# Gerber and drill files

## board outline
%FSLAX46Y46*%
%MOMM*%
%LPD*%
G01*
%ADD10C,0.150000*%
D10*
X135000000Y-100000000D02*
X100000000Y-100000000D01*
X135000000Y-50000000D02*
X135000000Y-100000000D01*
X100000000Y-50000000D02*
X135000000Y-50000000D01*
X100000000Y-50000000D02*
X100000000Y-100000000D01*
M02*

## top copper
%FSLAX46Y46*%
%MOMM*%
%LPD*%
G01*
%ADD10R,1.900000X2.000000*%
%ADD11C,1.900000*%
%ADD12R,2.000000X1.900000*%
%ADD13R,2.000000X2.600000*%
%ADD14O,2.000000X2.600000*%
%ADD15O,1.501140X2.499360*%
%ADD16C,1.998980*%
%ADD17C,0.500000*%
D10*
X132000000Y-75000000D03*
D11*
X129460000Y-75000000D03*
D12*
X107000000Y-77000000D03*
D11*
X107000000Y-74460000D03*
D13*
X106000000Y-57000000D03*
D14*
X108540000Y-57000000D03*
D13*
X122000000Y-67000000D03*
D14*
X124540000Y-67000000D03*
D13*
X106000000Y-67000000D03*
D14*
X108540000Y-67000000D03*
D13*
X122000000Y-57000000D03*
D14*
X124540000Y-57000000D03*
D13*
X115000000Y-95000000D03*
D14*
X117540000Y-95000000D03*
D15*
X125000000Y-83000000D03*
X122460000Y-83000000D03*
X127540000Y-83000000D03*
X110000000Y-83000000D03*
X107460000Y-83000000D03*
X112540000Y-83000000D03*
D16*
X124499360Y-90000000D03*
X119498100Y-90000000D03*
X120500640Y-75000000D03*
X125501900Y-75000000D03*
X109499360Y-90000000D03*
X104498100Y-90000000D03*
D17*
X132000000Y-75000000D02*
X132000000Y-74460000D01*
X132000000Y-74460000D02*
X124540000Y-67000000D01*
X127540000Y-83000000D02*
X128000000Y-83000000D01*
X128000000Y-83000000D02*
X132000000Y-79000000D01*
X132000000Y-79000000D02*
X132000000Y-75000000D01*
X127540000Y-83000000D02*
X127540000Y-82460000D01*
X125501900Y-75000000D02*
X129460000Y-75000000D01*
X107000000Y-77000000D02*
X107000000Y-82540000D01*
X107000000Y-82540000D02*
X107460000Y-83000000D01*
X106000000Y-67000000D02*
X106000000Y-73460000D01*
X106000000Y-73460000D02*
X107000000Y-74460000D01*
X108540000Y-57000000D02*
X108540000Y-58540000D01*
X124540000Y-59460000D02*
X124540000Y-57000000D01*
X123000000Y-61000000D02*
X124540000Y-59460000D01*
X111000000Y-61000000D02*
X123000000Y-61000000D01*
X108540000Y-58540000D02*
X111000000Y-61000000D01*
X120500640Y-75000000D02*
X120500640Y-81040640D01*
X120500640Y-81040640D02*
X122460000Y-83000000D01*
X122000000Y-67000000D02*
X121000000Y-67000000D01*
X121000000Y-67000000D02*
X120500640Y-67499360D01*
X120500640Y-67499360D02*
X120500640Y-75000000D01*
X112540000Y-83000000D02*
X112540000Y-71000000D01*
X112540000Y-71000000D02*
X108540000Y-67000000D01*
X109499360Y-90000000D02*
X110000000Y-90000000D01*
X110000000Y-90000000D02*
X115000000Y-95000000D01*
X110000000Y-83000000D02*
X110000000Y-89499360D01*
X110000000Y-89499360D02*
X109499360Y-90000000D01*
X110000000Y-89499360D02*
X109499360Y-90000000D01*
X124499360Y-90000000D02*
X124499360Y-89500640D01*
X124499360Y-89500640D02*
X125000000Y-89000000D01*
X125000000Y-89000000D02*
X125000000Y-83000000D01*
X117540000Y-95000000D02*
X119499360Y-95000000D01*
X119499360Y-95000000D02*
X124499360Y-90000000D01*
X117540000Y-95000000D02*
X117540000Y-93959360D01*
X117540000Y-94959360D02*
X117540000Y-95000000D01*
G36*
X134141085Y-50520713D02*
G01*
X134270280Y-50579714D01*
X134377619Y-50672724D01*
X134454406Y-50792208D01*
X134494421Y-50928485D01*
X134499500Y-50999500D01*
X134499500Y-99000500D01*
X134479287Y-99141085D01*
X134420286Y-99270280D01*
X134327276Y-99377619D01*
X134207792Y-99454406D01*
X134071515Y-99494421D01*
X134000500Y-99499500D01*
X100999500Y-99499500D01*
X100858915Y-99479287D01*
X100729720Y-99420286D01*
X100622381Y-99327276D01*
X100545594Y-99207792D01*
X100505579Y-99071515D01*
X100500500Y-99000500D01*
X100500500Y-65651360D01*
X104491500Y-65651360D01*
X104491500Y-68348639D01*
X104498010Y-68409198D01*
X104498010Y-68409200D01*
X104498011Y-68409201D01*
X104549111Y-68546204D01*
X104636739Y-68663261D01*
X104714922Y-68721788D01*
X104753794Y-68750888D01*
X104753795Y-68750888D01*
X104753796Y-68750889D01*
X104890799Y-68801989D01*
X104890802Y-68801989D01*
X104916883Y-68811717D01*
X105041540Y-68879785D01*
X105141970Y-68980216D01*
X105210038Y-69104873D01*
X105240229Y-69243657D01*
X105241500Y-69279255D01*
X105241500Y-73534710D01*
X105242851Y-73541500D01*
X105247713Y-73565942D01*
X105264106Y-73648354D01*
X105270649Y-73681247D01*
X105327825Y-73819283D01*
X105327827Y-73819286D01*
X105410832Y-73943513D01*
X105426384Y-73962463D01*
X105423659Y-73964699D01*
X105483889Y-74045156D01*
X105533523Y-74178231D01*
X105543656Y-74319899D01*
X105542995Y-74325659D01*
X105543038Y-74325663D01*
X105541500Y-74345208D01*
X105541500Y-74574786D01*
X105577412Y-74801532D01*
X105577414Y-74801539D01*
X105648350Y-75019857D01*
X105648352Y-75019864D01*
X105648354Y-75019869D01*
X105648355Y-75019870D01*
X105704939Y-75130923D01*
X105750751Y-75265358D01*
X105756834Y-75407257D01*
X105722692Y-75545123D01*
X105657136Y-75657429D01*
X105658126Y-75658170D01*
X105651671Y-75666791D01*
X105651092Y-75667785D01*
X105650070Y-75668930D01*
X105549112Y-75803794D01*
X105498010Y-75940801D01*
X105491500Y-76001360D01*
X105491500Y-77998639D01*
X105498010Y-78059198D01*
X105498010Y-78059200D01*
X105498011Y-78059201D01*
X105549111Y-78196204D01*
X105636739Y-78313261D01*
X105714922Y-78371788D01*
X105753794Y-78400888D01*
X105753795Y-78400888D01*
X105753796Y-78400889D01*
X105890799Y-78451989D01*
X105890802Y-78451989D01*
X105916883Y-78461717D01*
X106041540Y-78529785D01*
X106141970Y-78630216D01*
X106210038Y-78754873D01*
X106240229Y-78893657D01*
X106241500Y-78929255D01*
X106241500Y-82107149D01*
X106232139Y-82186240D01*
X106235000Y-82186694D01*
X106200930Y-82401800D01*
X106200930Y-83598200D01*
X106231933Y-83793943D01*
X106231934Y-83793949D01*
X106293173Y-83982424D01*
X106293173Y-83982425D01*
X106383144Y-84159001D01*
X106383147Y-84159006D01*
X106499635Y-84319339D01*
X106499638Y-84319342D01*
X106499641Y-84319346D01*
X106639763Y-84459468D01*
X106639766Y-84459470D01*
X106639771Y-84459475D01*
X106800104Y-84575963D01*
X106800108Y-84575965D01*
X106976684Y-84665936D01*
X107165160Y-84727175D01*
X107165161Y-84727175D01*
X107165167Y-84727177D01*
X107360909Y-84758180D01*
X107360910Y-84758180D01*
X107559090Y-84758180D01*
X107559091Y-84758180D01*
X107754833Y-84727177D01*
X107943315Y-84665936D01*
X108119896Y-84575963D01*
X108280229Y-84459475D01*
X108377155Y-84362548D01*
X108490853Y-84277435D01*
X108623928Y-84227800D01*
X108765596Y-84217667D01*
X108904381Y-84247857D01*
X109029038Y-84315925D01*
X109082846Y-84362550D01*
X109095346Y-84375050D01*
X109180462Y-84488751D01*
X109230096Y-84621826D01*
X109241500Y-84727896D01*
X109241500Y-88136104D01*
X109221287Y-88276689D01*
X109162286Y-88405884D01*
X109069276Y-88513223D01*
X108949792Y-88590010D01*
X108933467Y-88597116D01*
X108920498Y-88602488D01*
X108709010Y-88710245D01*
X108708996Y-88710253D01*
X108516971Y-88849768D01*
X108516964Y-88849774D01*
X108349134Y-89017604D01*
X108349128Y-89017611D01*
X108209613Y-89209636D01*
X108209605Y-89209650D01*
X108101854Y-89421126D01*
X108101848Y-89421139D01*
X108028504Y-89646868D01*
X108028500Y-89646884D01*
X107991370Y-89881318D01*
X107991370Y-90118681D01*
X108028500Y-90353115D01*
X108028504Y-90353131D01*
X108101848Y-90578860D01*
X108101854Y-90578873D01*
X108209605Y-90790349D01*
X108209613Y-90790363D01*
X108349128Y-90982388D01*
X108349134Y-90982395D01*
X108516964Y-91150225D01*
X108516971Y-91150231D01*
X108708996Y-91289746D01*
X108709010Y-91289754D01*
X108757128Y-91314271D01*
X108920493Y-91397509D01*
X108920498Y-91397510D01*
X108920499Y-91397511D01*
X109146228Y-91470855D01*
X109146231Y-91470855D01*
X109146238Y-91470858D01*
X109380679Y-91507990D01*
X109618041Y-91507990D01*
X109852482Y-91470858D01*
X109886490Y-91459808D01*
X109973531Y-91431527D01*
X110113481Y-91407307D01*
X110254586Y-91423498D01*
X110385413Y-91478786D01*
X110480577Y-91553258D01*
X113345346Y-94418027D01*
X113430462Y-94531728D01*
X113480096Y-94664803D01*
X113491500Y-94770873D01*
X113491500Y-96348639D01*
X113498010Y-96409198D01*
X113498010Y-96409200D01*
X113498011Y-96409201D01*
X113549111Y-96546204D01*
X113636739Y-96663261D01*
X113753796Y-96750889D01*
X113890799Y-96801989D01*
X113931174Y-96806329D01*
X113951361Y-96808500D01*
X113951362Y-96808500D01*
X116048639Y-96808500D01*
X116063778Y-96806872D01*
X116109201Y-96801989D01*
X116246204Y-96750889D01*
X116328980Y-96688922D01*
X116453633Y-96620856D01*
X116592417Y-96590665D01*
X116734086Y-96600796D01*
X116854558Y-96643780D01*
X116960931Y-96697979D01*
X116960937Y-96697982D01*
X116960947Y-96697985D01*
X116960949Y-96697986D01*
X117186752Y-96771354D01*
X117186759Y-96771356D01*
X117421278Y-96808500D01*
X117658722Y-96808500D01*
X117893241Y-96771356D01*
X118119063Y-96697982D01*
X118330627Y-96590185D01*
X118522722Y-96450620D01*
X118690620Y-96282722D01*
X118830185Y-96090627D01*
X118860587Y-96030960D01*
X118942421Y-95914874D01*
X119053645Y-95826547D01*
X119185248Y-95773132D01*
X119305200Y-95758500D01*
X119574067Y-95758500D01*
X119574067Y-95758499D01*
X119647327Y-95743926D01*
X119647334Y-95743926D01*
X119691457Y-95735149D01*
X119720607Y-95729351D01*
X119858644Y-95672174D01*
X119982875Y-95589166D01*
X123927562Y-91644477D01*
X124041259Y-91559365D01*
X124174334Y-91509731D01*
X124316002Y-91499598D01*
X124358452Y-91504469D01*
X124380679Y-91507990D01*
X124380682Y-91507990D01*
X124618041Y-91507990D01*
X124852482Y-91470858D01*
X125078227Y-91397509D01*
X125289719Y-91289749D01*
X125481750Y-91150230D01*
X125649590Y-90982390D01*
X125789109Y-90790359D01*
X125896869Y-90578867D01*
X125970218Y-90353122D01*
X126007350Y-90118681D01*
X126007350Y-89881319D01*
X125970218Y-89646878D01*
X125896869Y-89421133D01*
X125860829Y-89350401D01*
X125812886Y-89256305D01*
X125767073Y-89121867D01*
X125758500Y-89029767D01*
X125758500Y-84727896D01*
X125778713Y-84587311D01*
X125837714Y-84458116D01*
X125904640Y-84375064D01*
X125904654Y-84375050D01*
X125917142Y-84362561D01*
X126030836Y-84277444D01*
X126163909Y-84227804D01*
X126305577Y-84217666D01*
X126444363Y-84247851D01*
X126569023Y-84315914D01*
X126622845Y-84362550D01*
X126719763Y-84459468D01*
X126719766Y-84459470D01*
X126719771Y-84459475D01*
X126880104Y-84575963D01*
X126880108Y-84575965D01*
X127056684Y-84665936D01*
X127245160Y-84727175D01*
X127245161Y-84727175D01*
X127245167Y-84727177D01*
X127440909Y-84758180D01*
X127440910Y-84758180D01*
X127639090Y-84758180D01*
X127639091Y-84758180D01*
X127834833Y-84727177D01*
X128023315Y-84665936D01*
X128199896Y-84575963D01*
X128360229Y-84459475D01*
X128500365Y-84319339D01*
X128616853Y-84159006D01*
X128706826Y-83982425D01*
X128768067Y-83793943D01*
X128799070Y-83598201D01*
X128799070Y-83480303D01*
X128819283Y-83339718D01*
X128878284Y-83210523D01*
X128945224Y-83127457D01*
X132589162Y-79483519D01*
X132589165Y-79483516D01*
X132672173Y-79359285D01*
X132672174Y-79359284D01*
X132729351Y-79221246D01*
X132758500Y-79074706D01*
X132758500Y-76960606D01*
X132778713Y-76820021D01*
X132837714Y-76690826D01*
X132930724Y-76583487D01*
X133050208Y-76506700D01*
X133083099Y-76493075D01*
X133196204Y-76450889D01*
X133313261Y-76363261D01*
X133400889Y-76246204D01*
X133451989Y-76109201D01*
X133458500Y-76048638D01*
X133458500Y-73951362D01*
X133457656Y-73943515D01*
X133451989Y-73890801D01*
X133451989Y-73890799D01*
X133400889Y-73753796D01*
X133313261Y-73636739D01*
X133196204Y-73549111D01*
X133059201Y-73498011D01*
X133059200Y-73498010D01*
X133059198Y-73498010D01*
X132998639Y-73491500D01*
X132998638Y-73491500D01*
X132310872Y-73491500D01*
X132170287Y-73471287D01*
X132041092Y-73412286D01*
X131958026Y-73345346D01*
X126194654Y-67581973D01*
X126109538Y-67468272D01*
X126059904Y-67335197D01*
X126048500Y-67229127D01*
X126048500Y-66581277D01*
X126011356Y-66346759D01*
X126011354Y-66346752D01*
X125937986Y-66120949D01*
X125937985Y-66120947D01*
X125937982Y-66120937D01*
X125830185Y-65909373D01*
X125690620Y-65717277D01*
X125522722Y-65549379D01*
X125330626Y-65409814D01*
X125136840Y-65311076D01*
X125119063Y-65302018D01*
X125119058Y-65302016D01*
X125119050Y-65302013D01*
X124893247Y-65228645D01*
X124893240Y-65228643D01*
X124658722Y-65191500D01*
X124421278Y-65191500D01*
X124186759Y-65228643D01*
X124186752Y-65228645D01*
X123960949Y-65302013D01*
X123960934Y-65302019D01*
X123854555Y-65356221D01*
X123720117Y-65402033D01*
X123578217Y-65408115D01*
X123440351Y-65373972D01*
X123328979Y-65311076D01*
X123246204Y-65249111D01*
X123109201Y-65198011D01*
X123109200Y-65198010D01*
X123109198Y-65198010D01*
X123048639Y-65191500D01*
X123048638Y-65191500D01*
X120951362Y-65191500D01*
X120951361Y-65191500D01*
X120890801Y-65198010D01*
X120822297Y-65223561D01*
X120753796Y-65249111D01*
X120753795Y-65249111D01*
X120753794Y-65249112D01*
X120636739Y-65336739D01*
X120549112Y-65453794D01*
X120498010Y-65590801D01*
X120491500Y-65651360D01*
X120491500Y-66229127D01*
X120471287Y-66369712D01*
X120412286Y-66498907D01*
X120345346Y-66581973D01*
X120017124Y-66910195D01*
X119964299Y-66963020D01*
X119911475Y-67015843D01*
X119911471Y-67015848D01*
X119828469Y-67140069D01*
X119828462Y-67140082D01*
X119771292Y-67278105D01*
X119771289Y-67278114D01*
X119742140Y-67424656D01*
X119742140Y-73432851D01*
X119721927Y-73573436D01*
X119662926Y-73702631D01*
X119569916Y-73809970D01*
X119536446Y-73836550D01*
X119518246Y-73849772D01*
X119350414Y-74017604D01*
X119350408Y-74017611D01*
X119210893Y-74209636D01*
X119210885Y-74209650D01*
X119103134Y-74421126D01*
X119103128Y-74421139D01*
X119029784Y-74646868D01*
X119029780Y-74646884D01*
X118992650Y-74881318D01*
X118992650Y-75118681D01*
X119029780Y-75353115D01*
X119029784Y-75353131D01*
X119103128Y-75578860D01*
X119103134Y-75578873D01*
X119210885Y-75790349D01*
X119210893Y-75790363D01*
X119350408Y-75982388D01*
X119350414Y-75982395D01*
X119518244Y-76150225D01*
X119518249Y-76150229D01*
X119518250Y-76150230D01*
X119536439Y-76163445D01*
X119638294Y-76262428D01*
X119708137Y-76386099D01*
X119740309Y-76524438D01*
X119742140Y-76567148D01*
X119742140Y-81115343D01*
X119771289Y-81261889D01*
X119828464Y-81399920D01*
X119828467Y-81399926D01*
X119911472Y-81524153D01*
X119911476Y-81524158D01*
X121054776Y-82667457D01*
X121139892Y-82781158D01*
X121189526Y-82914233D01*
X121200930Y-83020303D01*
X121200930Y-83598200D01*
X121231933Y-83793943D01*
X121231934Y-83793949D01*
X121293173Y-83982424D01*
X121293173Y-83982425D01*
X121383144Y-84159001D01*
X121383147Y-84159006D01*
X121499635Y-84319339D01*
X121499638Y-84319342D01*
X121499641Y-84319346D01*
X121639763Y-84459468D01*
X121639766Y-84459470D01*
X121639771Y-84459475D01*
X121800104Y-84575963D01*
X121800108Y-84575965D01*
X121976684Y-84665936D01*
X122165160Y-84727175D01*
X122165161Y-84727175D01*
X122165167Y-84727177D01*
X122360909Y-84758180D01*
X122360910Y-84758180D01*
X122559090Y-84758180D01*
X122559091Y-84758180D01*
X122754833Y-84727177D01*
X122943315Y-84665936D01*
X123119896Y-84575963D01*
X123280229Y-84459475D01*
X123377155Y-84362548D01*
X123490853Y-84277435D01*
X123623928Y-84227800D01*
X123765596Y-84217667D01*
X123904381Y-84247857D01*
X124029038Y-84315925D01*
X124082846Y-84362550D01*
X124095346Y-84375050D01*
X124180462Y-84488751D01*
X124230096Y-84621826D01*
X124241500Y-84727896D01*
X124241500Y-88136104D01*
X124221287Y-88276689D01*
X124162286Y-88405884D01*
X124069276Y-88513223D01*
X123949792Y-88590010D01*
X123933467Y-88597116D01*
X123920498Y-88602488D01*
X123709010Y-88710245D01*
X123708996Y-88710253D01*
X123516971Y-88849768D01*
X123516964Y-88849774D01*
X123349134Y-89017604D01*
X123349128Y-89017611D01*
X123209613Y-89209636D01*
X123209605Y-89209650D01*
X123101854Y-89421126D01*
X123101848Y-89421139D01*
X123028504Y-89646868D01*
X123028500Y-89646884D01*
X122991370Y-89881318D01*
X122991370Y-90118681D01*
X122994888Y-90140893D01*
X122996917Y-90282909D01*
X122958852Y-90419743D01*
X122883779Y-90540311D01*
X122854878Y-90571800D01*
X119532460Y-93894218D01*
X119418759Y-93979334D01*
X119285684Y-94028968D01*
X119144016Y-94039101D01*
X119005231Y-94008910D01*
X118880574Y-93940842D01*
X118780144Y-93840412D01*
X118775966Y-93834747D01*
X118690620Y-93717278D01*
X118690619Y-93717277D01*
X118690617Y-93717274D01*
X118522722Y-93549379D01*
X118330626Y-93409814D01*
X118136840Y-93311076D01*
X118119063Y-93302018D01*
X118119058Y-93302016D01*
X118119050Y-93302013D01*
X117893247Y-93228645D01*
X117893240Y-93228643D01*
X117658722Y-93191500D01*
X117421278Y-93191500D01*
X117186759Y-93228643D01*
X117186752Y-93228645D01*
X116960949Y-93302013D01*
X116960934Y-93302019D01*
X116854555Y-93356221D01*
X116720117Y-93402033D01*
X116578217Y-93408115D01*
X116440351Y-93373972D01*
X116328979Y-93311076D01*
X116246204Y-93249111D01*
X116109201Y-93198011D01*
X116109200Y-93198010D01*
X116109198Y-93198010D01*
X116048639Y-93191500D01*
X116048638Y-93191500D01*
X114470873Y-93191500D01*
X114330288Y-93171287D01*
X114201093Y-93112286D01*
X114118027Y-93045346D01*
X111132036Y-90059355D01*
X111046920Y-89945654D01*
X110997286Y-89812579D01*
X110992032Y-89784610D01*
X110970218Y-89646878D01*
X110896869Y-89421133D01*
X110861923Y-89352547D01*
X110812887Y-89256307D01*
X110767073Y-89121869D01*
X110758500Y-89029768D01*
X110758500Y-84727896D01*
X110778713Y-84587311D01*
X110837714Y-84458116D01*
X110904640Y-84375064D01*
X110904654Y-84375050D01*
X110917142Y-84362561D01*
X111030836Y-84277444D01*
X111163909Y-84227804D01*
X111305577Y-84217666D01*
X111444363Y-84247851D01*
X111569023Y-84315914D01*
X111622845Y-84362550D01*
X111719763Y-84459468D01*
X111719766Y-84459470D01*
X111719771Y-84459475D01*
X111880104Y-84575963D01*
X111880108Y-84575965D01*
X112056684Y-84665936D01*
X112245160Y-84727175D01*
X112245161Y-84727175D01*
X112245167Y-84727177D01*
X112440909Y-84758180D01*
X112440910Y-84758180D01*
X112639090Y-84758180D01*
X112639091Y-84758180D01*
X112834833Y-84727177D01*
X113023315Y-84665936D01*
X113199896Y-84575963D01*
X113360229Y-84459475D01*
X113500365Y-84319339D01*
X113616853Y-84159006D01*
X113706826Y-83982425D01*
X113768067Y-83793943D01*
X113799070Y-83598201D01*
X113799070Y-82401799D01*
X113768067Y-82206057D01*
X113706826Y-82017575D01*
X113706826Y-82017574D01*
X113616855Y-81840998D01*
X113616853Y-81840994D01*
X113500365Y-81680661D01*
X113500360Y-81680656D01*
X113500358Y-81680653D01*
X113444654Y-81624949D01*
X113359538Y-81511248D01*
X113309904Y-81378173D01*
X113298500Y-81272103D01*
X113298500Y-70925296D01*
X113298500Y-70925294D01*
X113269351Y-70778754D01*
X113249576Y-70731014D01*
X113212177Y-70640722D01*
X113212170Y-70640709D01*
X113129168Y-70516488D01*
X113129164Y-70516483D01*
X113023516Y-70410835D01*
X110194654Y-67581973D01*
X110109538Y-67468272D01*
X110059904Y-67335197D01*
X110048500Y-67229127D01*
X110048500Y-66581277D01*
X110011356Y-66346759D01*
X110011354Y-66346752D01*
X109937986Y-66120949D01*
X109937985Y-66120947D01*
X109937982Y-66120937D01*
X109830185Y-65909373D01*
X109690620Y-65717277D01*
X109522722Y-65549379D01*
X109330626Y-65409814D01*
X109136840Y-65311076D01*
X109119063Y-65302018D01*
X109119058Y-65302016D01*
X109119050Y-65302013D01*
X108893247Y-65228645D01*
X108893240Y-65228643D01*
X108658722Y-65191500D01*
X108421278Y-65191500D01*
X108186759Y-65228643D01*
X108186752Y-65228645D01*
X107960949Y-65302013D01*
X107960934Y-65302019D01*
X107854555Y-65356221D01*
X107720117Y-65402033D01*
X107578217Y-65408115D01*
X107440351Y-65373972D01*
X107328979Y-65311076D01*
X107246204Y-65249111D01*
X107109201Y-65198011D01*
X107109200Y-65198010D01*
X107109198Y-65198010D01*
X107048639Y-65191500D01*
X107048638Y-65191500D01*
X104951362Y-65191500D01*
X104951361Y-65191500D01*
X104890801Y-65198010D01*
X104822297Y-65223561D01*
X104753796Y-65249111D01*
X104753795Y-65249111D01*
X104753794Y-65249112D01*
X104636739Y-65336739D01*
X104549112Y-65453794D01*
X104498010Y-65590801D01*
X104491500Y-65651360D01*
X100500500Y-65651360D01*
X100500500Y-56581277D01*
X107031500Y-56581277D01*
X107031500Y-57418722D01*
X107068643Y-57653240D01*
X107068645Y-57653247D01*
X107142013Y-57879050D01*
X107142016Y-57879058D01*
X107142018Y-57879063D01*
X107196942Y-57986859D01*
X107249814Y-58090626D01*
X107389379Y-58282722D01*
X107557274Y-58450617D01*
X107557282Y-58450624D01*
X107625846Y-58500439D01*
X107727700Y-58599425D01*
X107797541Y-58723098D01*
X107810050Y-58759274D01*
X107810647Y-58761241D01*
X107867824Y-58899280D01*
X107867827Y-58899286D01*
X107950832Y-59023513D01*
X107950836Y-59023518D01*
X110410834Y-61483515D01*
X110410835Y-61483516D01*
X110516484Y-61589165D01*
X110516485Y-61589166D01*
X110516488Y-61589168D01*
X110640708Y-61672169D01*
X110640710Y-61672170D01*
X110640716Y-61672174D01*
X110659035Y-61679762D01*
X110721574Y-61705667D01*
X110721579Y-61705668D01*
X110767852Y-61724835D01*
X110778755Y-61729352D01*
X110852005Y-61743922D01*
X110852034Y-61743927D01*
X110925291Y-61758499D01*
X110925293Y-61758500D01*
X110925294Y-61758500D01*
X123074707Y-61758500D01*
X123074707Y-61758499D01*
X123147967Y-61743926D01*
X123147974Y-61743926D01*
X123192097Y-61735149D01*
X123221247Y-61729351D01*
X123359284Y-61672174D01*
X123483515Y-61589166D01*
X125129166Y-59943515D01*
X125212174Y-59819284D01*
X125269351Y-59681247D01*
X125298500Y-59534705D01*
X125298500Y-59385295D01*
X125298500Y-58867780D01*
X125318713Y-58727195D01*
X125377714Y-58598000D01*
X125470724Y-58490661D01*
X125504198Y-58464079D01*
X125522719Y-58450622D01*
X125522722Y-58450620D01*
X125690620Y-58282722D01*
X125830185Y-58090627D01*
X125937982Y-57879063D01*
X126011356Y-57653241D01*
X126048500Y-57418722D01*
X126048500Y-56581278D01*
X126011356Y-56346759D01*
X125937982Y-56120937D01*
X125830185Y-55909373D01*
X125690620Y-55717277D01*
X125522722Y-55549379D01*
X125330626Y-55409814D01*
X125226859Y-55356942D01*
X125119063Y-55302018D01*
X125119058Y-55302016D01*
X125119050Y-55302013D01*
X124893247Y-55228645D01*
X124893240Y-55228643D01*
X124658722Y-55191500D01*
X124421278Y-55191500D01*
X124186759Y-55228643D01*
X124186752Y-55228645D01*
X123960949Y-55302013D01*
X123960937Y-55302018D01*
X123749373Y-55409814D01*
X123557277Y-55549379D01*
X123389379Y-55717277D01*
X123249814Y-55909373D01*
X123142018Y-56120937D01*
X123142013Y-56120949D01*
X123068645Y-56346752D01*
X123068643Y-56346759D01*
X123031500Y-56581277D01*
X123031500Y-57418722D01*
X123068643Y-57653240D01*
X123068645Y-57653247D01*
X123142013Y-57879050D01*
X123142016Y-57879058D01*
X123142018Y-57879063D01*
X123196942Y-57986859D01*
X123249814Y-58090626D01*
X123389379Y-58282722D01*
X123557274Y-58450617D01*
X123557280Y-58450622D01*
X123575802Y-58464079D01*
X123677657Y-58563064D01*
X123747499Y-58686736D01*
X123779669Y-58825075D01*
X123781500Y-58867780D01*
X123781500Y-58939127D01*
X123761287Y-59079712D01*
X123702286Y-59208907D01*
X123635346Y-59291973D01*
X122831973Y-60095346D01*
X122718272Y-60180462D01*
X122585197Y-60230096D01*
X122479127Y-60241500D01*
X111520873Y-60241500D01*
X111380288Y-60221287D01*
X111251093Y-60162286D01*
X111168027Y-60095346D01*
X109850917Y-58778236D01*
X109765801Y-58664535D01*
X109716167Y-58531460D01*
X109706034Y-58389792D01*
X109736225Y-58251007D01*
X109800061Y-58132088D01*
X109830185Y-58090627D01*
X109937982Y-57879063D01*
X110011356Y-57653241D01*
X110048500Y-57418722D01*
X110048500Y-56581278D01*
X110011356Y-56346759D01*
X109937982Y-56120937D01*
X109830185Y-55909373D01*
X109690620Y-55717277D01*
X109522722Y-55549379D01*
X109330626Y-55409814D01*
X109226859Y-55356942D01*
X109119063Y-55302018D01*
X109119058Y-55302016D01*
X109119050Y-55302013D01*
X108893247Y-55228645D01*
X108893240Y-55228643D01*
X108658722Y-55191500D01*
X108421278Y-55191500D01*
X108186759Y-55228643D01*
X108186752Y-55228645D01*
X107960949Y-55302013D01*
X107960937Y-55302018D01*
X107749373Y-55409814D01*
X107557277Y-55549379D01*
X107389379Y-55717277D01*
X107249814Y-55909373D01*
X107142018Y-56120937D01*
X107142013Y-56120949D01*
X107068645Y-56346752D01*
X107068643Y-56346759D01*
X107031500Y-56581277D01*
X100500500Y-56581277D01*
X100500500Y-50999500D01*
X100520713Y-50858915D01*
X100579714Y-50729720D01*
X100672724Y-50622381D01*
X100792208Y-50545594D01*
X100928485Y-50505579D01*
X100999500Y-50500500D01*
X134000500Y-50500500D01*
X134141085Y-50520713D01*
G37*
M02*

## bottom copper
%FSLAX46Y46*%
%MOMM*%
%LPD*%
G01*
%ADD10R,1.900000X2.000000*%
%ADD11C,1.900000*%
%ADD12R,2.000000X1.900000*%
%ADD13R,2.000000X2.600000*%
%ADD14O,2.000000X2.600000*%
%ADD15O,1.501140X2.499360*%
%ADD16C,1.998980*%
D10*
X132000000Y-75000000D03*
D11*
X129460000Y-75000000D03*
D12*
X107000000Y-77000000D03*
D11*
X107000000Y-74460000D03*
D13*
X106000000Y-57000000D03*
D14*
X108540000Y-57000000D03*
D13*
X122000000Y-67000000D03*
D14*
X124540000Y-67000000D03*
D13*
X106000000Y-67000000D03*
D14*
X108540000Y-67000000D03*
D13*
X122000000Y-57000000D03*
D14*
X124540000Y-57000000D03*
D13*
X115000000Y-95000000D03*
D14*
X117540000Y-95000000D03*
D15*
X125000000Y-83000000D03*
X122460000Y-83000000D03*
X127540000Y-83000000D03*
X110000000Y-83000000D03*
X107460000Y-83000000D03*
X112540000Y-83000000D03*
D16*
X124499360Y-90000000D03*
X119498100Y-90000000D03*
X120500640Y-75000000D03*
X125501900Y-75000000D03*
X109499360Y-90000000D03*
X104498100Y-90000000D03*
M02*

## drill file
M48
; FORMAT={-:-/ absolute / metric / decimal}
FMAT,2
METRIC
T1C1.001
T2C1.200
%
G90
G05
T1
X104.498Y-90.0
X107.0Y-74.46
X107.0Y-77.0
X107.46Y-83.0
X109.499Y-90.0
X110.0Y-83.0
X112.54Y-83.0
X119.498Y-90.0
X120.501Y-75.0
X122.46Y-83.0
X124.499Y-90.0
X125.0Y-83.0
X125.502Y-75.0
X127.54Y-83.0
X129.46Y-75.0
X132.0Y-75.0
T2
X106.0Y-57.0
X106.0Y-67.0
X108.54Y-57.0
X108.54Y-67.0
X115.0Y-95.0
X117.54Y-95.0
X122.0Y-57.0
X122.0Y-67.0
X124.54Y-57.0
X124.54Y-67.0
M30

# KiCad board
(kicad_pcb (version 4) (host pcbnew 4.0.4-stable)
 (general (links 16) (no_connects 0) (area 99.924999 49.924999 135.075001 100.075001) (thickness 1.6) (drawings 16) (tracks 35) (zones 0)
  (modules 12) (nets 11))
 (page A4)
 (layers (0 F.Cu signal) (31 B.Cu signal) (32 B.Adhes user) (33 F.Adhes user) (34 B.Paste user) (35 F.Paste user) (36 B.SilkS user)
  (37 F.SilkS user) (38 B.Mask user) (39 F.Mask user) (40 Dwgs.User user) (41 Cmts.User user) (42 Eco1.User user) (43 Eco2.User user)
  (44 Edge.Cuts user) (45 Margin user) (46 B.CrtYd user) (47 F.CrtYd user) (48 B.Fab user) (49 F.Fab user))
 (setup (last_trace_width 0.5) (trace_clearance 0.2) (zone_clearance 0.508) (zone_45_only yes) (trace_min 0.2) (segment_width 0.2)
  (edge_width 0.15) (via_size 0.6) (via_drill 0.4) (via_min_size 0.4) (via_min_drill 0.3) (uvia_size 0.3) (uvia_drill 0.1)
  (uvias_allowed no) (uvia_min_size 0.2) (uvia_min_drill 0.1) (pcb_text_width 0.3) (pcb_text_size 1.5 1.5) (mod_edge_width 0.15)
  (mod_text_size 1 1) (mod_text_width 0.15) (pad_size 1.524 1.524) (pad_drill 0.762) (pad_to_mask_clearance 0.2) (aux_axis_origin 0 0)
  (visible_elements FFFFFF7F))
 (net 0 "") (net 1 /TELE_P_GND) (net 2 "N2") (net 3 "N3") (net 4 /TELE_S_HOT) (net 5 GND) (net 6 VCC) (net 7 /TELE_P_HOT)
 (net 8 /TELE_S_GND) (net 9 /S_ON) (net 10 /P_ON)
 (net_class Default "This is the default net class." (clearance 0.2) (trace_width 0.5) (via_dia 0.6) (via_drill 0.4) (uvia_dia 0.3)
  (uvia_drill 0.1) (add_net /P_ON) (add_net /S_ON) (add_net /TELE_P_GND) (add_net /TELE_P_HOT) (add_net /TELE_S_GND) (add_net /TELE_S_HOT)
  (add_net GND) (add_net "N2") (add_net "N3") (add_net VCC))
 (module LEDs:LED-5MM (layer F.Cu) (at 132 75 180)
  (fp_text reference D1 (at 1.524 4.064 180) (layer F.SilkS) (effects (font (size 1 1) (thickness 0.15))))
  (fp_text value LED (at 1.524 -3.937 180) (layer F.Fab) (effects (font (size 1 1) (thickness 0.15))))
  (pad 1 thru_hole rect (at 0 0 270) (size 2 1.9) (drill 1.00076) (layers *.Cu *.Mask) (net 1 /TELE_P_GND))
  (pad 2 thru_hole circle (at 2.54 0 180) (size 1.9 1.9) (drill 1.00076) (layers *.Cu *.Mask) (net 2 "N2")))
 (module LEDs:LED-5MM (layer F.Cu) (at 107 77 90)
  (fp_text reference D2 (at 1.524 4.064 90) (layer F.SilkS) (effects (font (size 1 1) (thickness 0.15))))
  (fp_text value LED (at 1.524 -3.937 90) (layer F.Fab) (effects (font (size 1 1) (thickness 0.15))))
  (pad 1 thru_hole rect (at 0 0 180) (size 2 1.9) (drill 1.00076) (layers *.Cu *.Mask) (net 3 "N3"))
  (pad 2 thru_hole circle (at 2.54 0 90) (size 1.9 1.9) (drill 1.00076) (layers *.Cu *.Mask) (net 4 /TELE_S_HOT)))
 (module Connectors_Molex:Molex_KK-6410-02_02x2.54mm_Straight (layer F.Cu) (at 106 57)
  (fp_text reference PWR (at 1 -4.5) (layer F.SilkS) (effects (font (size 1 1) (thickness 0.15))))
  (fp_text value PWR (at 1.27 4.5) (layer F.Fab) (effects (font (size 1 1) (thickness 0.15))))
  (pad 1 thru_hole rect (at 0 0) (size 2 2.6) (drill 1.2) (layers *.Cu *.Mask) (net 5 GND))
  (pad 2 thru_hole oval (at 2.54 0) (size 2 2.6) (drill 1.2) (layers *.Cu *.Mask) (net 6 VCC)))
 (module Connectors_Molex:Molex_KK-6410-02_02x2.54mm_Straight (layer F.Cu) (at 122 67)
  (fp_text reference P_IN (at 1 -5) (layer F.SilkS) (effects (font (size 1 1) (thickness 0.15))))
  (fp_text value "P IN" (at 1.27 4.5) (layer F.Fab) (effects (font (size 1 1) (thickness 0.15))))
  (pad 1 thru_hole rect (at 0 0) (size 2 2.6) (drill 1.2) (layers *.Cu *.Mask) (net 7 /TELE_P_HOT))
  (pad 2 thru_hole oval (at 2.54 0) (size 2 2.6) (drill 1.2) (layers *.Cu *.Mask) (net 1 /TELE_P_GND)))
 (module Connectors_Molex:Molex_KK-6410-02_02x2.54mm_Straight (layer F.Cu) (at 106 67)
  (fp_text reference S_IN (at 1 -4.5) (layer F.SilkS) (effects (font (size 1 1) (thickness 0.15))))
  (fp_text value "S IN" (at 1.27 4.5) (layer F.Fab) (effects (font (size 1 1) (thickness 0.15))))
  (pad 1 thru_hole rect (at 0 0) (size 2 2.6) (drill 1.2) (layers *.Cu *.Mask) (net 4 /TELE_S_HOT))
  (pad 2 thru_hole oval (at 2.54 0) (size 2 2.6) (drill 1.2) (layers *.Cu *.Mask) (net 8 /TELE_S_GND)))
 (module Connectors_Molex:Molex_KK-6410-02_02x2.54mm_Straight (layer F.Cu) (at 122 57)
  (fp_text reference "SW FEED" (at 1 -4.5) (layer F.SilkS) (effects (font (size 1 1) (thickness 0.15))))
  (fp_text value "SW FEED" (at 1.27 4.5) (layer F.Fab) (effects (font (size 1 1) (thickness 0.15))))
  (pad 1 thru_hole rect (at 0 0) (size 2 2.6) (drill 1.2) (layers *.Cu *.Mask) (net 5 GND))
  (pad 2 thru_hole oval (at 2.54 0) (size 2 2.6) (drill 1.2) (layers *.Cu *.Mask) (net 6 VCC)))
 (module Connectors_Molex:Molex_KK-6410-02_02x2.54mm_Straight (layer F.Cu) (at 115 95)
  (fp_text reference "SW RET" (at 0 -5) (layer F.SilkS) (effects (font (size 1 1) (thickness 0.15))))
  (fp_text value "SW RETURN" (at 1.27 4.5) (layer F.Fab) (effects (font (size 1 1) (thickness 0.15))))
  (pad 1 thru_hole rect (at 0 0) (size 2 2.6) (drill 1.2) (layers *.Cu *.Mask) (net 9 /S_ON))
  (pad 2 thru_hole oval (at 2.54 0) (size 2 2.6) (drill 1.2) (layers *.Cu *.Mask) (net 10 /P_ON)))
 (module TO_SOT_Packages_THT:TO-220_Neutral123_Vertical (layer F.Cu) (at 125 83)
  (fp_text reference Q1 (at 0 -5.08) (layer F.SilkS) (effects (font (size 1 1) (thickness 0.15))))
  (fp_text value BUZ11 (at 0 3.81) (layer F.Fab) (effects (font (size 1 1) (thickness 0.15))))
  (pad 2 thru_hole oval (at 0 0 90) (size 2.49936 1.50114) (drill 1.00076) (layers *.Cu *.Mask) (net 10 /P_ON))
  (pad 1 thru_hole oval (at -2.54 0 90) (size 2.49936 1.50114) (drill 1.00076) (layers *.Cu *.Mask) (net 7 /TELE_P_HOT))
  (pad 3 thru_hole oval (at 2.54 0 90) (size 2.49936 1.50114) (drill 1.00076) (layers *.Cu *.Mask) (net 1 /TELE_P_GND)))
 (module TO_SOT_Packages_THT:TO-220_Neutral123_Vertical (layer F.Cu) (at 110 83)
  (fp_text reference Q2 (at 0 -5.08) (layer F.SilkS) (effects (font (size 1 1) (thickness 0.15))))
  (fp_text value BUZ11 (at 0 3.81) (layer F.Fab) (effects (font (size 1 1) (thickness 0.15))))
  (pad 2 thru_hole oval (at 0 0 90) (size 2.49936 1.50114) (drill 1.00076) (layers *.Cu *.Mask) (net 9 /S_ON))
  (pad 1 thru_hole oval (at -2.54 0 90) (size 2.49936 1.50114) (drill 1.00076) (layers *.Cu *.Mask) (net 3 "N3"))
  (pad 3 thru_hole oval (at 2.54 0 90) (size 2.49936 1.50114) (drill 1.00076) (layers *.Cu *.Mask) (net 8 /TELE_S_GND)))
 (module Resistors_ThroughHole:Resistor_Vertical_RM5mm (layer F.Cu) (at 122 90 180)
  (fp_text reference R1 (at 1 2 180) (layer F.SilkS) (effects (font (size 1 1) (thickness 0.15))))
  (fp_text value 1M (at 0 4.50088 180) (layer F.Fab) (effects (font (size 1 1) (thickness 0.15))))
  (pad 1 thru_hole circle (at -2.49936 0 180) (size 1.99898 1.99898) (drill 1.00076) (layers *.Cu *.SilkS *.Mask) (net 10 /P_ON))
  (pad 2 thru_hole circle (at 2.5019 0 180) (size 1.99898 1.99898) (drill 1.00076) (layers *.Cu *.SilkS *.Mask) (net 5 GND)))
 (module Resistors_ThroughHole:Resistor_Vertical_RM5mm (layer F.Cu) (at 123 75)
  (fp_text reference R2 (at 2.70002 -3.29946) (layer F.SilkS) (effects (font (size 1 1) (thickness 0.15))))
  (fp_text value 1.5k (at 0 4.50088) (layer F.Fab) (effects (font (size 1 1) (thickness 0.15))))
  (pad 1 thru_hole circle (at -2.49936 0) (size 1.99898 1.99898) (drill 1.00076) (layers *.Cu *.SilkS *.Mask) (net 7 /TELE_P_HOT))
  (pad 2 thru_hole circle (at 2.5019 0) (size 1.99898 1.99898) (drill 1.00076) (layers *.Cu *.SilkS *.Mask) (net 2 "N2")))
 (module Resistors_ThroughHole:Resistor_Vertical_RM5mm (layer F.Cu) (at 107 90 180)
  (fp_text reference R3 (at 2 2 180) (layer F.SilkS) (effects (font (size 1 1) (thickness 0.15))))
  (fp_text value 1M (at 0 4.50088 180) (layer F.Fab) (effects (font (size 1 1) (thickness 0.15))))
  (pad 1 thru_hole circle (at -2.49936 0 180) (size 1.99898 1.99898) (drill 1.00076) (layers *.Cu *.SilkS *.Mask) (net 9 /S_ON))
  (pad 2 thru_hole circle (at 2.5019 0 180) (size 1.99898 1.99898) (drill 1.00076) (layers *.Cu *.SilkS *.Mask) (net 5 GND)))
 (gr_line (start 135 100) (end 100 100) (angle 90) (layer Edge.Cuts) (width 0.15))
 (gr_line (start 135 50) (end 135 100) (angle 90) (layer Edge.Cuts) (width 0.15))
 (gr_line (start 100 50) (end 135 50) (angle 90) (layer Edge.Cuts) (width 0.15))
 (gr_line (start 100 50) (end 100 100) (angle 90) (layer Edge.Cuts) (width 0.15))
 (segment (start 132 75) (end 132 74.46) (width 0.5) (layer F.Cu) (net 1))
 (segment (start 132 74.46) (end 124.54 67) (width 0.5) (layer F.Cu) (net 1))
 (segment (start 127.54 83) (end 128 83) (width 0.5) (layer F.Cu) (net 1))
 (segment (start 128 83) (end 132 79) (width 0.5) (layer F.Cu) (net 1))
 (segment (start 132 79) (end 132 75) (width 0.5) (layer F.Cu) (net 1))
 (segment (start 127.54 83) (end 127.54 82.46) (width 0.5) (layer F.Cu) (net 1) (status 30))
 (segment (start 125.5019 75) (end 129.46 75) (width 0.5) (layer F.Cu) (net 2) (status 30))
 (segment (start 107 77) (end 107 82.54) (width 0.5) (layer F.Cu) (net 3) (status 30))
 (segment (start 107 82.54) (end 107.46 83) (width 0.5) (layer F.Cu) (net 3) (status 30))
 (segment (start 106 67) (end 106 73.46) (width 0.5) (layer F.Cu) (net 4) (status 10))
 (segment (start 106 73.46) (end 107 74.46) (width 0.5) (layer F.Cu) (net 4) (status 20))
 (segment (start 108.54 57) (end 108.54 58.54) (width 0.5) (layer F.Cu) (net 6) (status 400000))
 (segment (start 124.54 59.46) (end 124.54 57) (width 0.5) (layer F.Cu) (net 6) (status 800000))
 (segment (start 123 61) (end 124.54 59.46) (width 0.5) (layer F.Cu) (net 6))
 (segment (start 111 61) (end 123 61) (width 0.5) (layer F.Cu) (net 6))
 (segment (start 108.54 58.54) (end 111 61) (width 0.5) (layer F.Cu) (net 6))
 (segment (start 120.50064 75) (end 120.50064 81.04064) (width 0.5) (layer F.Cu) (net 7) (status 10))
 (segment (start 120.50064 81.04064) (end 122.46 83) (width 0.5) (layer F.Cu) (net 7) (status 20))
 (segment (start 122 67) (end 121 67) (width 0.5) (layer F.Cu) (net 7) (status 30))
 (segment (start 121 67) (end 120.50064 67.49936) (width 0.5) (layer F.Cu) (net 7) (status 10))
 (segment (start 120.50064 67.49936) (end 120.50064 75) (width 0.5) (layer F.Cu) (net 7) (status 20))
 (segment (start 112.54 83) (end 112.54 71) (width 0.5) (layer F.Cu) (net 8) (status 10))
 (segment (start 112.54 71) (end 108.54 67) (width 0.5) (layer F.Cu) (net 8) (status 20))
 (segment (start 109.49936 90) (end 110 90) (width 0.5) (layer F.Cu) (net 9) (status 30))
 (segment (start 110 90) (end 115 95) (width 0.5) (layer F.Cu) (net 9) (status 30))
 (segment (start 110 83) (end 110 89.49936) (width 0.5) (layer F.Cu) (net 9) (status 30))
 (segment (start 110 89.49936) (end 109.49936 90) (width 0.5) (layer F.Cu) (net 9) (status 30))
 (segment (start 110 89.49936) (end 109.49936 90) (width 0.5) (layer F.Cu) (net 9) (status 30))
 (segment (start 124.49936 90) (end 124.49936 89.50064) (width 0.5) (layer F.Cu) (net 10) (status 30))
 (segment (start 124.49936 89.50064) (end 125 89) (width 0.5) (layer F.Cu) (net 10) (status 10))
 (segment (start 125 89) (end 125 83) (width 0.5) (layer F.Cu) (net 10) (status 20))
 (segment (start 117.54 95) (end 119.49936 95) (width 0.5) (layer F.Cu) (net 10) (status 10))
 (segment (start 119.49936 95) (end 124.49936 90) (width 0.5) (layer F.Cu) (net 10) (status 20))
 (segment (start 117.54 95) (end 117.54 93.95936) (width 0.5) (layer F.Cu) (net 10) (status 30))
 (segment (start 117.54 94.95936) (end 117.54 95) (width 0.5) (layer F.Cu) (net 10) (status 30))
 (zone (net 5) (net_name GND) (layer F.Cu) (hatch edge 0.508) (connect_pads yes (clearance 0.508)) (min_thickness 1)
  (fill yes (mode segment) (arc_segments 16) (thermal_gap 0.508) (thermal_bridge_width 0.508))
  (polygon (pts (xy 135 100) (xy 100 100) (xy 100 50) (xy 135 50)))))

